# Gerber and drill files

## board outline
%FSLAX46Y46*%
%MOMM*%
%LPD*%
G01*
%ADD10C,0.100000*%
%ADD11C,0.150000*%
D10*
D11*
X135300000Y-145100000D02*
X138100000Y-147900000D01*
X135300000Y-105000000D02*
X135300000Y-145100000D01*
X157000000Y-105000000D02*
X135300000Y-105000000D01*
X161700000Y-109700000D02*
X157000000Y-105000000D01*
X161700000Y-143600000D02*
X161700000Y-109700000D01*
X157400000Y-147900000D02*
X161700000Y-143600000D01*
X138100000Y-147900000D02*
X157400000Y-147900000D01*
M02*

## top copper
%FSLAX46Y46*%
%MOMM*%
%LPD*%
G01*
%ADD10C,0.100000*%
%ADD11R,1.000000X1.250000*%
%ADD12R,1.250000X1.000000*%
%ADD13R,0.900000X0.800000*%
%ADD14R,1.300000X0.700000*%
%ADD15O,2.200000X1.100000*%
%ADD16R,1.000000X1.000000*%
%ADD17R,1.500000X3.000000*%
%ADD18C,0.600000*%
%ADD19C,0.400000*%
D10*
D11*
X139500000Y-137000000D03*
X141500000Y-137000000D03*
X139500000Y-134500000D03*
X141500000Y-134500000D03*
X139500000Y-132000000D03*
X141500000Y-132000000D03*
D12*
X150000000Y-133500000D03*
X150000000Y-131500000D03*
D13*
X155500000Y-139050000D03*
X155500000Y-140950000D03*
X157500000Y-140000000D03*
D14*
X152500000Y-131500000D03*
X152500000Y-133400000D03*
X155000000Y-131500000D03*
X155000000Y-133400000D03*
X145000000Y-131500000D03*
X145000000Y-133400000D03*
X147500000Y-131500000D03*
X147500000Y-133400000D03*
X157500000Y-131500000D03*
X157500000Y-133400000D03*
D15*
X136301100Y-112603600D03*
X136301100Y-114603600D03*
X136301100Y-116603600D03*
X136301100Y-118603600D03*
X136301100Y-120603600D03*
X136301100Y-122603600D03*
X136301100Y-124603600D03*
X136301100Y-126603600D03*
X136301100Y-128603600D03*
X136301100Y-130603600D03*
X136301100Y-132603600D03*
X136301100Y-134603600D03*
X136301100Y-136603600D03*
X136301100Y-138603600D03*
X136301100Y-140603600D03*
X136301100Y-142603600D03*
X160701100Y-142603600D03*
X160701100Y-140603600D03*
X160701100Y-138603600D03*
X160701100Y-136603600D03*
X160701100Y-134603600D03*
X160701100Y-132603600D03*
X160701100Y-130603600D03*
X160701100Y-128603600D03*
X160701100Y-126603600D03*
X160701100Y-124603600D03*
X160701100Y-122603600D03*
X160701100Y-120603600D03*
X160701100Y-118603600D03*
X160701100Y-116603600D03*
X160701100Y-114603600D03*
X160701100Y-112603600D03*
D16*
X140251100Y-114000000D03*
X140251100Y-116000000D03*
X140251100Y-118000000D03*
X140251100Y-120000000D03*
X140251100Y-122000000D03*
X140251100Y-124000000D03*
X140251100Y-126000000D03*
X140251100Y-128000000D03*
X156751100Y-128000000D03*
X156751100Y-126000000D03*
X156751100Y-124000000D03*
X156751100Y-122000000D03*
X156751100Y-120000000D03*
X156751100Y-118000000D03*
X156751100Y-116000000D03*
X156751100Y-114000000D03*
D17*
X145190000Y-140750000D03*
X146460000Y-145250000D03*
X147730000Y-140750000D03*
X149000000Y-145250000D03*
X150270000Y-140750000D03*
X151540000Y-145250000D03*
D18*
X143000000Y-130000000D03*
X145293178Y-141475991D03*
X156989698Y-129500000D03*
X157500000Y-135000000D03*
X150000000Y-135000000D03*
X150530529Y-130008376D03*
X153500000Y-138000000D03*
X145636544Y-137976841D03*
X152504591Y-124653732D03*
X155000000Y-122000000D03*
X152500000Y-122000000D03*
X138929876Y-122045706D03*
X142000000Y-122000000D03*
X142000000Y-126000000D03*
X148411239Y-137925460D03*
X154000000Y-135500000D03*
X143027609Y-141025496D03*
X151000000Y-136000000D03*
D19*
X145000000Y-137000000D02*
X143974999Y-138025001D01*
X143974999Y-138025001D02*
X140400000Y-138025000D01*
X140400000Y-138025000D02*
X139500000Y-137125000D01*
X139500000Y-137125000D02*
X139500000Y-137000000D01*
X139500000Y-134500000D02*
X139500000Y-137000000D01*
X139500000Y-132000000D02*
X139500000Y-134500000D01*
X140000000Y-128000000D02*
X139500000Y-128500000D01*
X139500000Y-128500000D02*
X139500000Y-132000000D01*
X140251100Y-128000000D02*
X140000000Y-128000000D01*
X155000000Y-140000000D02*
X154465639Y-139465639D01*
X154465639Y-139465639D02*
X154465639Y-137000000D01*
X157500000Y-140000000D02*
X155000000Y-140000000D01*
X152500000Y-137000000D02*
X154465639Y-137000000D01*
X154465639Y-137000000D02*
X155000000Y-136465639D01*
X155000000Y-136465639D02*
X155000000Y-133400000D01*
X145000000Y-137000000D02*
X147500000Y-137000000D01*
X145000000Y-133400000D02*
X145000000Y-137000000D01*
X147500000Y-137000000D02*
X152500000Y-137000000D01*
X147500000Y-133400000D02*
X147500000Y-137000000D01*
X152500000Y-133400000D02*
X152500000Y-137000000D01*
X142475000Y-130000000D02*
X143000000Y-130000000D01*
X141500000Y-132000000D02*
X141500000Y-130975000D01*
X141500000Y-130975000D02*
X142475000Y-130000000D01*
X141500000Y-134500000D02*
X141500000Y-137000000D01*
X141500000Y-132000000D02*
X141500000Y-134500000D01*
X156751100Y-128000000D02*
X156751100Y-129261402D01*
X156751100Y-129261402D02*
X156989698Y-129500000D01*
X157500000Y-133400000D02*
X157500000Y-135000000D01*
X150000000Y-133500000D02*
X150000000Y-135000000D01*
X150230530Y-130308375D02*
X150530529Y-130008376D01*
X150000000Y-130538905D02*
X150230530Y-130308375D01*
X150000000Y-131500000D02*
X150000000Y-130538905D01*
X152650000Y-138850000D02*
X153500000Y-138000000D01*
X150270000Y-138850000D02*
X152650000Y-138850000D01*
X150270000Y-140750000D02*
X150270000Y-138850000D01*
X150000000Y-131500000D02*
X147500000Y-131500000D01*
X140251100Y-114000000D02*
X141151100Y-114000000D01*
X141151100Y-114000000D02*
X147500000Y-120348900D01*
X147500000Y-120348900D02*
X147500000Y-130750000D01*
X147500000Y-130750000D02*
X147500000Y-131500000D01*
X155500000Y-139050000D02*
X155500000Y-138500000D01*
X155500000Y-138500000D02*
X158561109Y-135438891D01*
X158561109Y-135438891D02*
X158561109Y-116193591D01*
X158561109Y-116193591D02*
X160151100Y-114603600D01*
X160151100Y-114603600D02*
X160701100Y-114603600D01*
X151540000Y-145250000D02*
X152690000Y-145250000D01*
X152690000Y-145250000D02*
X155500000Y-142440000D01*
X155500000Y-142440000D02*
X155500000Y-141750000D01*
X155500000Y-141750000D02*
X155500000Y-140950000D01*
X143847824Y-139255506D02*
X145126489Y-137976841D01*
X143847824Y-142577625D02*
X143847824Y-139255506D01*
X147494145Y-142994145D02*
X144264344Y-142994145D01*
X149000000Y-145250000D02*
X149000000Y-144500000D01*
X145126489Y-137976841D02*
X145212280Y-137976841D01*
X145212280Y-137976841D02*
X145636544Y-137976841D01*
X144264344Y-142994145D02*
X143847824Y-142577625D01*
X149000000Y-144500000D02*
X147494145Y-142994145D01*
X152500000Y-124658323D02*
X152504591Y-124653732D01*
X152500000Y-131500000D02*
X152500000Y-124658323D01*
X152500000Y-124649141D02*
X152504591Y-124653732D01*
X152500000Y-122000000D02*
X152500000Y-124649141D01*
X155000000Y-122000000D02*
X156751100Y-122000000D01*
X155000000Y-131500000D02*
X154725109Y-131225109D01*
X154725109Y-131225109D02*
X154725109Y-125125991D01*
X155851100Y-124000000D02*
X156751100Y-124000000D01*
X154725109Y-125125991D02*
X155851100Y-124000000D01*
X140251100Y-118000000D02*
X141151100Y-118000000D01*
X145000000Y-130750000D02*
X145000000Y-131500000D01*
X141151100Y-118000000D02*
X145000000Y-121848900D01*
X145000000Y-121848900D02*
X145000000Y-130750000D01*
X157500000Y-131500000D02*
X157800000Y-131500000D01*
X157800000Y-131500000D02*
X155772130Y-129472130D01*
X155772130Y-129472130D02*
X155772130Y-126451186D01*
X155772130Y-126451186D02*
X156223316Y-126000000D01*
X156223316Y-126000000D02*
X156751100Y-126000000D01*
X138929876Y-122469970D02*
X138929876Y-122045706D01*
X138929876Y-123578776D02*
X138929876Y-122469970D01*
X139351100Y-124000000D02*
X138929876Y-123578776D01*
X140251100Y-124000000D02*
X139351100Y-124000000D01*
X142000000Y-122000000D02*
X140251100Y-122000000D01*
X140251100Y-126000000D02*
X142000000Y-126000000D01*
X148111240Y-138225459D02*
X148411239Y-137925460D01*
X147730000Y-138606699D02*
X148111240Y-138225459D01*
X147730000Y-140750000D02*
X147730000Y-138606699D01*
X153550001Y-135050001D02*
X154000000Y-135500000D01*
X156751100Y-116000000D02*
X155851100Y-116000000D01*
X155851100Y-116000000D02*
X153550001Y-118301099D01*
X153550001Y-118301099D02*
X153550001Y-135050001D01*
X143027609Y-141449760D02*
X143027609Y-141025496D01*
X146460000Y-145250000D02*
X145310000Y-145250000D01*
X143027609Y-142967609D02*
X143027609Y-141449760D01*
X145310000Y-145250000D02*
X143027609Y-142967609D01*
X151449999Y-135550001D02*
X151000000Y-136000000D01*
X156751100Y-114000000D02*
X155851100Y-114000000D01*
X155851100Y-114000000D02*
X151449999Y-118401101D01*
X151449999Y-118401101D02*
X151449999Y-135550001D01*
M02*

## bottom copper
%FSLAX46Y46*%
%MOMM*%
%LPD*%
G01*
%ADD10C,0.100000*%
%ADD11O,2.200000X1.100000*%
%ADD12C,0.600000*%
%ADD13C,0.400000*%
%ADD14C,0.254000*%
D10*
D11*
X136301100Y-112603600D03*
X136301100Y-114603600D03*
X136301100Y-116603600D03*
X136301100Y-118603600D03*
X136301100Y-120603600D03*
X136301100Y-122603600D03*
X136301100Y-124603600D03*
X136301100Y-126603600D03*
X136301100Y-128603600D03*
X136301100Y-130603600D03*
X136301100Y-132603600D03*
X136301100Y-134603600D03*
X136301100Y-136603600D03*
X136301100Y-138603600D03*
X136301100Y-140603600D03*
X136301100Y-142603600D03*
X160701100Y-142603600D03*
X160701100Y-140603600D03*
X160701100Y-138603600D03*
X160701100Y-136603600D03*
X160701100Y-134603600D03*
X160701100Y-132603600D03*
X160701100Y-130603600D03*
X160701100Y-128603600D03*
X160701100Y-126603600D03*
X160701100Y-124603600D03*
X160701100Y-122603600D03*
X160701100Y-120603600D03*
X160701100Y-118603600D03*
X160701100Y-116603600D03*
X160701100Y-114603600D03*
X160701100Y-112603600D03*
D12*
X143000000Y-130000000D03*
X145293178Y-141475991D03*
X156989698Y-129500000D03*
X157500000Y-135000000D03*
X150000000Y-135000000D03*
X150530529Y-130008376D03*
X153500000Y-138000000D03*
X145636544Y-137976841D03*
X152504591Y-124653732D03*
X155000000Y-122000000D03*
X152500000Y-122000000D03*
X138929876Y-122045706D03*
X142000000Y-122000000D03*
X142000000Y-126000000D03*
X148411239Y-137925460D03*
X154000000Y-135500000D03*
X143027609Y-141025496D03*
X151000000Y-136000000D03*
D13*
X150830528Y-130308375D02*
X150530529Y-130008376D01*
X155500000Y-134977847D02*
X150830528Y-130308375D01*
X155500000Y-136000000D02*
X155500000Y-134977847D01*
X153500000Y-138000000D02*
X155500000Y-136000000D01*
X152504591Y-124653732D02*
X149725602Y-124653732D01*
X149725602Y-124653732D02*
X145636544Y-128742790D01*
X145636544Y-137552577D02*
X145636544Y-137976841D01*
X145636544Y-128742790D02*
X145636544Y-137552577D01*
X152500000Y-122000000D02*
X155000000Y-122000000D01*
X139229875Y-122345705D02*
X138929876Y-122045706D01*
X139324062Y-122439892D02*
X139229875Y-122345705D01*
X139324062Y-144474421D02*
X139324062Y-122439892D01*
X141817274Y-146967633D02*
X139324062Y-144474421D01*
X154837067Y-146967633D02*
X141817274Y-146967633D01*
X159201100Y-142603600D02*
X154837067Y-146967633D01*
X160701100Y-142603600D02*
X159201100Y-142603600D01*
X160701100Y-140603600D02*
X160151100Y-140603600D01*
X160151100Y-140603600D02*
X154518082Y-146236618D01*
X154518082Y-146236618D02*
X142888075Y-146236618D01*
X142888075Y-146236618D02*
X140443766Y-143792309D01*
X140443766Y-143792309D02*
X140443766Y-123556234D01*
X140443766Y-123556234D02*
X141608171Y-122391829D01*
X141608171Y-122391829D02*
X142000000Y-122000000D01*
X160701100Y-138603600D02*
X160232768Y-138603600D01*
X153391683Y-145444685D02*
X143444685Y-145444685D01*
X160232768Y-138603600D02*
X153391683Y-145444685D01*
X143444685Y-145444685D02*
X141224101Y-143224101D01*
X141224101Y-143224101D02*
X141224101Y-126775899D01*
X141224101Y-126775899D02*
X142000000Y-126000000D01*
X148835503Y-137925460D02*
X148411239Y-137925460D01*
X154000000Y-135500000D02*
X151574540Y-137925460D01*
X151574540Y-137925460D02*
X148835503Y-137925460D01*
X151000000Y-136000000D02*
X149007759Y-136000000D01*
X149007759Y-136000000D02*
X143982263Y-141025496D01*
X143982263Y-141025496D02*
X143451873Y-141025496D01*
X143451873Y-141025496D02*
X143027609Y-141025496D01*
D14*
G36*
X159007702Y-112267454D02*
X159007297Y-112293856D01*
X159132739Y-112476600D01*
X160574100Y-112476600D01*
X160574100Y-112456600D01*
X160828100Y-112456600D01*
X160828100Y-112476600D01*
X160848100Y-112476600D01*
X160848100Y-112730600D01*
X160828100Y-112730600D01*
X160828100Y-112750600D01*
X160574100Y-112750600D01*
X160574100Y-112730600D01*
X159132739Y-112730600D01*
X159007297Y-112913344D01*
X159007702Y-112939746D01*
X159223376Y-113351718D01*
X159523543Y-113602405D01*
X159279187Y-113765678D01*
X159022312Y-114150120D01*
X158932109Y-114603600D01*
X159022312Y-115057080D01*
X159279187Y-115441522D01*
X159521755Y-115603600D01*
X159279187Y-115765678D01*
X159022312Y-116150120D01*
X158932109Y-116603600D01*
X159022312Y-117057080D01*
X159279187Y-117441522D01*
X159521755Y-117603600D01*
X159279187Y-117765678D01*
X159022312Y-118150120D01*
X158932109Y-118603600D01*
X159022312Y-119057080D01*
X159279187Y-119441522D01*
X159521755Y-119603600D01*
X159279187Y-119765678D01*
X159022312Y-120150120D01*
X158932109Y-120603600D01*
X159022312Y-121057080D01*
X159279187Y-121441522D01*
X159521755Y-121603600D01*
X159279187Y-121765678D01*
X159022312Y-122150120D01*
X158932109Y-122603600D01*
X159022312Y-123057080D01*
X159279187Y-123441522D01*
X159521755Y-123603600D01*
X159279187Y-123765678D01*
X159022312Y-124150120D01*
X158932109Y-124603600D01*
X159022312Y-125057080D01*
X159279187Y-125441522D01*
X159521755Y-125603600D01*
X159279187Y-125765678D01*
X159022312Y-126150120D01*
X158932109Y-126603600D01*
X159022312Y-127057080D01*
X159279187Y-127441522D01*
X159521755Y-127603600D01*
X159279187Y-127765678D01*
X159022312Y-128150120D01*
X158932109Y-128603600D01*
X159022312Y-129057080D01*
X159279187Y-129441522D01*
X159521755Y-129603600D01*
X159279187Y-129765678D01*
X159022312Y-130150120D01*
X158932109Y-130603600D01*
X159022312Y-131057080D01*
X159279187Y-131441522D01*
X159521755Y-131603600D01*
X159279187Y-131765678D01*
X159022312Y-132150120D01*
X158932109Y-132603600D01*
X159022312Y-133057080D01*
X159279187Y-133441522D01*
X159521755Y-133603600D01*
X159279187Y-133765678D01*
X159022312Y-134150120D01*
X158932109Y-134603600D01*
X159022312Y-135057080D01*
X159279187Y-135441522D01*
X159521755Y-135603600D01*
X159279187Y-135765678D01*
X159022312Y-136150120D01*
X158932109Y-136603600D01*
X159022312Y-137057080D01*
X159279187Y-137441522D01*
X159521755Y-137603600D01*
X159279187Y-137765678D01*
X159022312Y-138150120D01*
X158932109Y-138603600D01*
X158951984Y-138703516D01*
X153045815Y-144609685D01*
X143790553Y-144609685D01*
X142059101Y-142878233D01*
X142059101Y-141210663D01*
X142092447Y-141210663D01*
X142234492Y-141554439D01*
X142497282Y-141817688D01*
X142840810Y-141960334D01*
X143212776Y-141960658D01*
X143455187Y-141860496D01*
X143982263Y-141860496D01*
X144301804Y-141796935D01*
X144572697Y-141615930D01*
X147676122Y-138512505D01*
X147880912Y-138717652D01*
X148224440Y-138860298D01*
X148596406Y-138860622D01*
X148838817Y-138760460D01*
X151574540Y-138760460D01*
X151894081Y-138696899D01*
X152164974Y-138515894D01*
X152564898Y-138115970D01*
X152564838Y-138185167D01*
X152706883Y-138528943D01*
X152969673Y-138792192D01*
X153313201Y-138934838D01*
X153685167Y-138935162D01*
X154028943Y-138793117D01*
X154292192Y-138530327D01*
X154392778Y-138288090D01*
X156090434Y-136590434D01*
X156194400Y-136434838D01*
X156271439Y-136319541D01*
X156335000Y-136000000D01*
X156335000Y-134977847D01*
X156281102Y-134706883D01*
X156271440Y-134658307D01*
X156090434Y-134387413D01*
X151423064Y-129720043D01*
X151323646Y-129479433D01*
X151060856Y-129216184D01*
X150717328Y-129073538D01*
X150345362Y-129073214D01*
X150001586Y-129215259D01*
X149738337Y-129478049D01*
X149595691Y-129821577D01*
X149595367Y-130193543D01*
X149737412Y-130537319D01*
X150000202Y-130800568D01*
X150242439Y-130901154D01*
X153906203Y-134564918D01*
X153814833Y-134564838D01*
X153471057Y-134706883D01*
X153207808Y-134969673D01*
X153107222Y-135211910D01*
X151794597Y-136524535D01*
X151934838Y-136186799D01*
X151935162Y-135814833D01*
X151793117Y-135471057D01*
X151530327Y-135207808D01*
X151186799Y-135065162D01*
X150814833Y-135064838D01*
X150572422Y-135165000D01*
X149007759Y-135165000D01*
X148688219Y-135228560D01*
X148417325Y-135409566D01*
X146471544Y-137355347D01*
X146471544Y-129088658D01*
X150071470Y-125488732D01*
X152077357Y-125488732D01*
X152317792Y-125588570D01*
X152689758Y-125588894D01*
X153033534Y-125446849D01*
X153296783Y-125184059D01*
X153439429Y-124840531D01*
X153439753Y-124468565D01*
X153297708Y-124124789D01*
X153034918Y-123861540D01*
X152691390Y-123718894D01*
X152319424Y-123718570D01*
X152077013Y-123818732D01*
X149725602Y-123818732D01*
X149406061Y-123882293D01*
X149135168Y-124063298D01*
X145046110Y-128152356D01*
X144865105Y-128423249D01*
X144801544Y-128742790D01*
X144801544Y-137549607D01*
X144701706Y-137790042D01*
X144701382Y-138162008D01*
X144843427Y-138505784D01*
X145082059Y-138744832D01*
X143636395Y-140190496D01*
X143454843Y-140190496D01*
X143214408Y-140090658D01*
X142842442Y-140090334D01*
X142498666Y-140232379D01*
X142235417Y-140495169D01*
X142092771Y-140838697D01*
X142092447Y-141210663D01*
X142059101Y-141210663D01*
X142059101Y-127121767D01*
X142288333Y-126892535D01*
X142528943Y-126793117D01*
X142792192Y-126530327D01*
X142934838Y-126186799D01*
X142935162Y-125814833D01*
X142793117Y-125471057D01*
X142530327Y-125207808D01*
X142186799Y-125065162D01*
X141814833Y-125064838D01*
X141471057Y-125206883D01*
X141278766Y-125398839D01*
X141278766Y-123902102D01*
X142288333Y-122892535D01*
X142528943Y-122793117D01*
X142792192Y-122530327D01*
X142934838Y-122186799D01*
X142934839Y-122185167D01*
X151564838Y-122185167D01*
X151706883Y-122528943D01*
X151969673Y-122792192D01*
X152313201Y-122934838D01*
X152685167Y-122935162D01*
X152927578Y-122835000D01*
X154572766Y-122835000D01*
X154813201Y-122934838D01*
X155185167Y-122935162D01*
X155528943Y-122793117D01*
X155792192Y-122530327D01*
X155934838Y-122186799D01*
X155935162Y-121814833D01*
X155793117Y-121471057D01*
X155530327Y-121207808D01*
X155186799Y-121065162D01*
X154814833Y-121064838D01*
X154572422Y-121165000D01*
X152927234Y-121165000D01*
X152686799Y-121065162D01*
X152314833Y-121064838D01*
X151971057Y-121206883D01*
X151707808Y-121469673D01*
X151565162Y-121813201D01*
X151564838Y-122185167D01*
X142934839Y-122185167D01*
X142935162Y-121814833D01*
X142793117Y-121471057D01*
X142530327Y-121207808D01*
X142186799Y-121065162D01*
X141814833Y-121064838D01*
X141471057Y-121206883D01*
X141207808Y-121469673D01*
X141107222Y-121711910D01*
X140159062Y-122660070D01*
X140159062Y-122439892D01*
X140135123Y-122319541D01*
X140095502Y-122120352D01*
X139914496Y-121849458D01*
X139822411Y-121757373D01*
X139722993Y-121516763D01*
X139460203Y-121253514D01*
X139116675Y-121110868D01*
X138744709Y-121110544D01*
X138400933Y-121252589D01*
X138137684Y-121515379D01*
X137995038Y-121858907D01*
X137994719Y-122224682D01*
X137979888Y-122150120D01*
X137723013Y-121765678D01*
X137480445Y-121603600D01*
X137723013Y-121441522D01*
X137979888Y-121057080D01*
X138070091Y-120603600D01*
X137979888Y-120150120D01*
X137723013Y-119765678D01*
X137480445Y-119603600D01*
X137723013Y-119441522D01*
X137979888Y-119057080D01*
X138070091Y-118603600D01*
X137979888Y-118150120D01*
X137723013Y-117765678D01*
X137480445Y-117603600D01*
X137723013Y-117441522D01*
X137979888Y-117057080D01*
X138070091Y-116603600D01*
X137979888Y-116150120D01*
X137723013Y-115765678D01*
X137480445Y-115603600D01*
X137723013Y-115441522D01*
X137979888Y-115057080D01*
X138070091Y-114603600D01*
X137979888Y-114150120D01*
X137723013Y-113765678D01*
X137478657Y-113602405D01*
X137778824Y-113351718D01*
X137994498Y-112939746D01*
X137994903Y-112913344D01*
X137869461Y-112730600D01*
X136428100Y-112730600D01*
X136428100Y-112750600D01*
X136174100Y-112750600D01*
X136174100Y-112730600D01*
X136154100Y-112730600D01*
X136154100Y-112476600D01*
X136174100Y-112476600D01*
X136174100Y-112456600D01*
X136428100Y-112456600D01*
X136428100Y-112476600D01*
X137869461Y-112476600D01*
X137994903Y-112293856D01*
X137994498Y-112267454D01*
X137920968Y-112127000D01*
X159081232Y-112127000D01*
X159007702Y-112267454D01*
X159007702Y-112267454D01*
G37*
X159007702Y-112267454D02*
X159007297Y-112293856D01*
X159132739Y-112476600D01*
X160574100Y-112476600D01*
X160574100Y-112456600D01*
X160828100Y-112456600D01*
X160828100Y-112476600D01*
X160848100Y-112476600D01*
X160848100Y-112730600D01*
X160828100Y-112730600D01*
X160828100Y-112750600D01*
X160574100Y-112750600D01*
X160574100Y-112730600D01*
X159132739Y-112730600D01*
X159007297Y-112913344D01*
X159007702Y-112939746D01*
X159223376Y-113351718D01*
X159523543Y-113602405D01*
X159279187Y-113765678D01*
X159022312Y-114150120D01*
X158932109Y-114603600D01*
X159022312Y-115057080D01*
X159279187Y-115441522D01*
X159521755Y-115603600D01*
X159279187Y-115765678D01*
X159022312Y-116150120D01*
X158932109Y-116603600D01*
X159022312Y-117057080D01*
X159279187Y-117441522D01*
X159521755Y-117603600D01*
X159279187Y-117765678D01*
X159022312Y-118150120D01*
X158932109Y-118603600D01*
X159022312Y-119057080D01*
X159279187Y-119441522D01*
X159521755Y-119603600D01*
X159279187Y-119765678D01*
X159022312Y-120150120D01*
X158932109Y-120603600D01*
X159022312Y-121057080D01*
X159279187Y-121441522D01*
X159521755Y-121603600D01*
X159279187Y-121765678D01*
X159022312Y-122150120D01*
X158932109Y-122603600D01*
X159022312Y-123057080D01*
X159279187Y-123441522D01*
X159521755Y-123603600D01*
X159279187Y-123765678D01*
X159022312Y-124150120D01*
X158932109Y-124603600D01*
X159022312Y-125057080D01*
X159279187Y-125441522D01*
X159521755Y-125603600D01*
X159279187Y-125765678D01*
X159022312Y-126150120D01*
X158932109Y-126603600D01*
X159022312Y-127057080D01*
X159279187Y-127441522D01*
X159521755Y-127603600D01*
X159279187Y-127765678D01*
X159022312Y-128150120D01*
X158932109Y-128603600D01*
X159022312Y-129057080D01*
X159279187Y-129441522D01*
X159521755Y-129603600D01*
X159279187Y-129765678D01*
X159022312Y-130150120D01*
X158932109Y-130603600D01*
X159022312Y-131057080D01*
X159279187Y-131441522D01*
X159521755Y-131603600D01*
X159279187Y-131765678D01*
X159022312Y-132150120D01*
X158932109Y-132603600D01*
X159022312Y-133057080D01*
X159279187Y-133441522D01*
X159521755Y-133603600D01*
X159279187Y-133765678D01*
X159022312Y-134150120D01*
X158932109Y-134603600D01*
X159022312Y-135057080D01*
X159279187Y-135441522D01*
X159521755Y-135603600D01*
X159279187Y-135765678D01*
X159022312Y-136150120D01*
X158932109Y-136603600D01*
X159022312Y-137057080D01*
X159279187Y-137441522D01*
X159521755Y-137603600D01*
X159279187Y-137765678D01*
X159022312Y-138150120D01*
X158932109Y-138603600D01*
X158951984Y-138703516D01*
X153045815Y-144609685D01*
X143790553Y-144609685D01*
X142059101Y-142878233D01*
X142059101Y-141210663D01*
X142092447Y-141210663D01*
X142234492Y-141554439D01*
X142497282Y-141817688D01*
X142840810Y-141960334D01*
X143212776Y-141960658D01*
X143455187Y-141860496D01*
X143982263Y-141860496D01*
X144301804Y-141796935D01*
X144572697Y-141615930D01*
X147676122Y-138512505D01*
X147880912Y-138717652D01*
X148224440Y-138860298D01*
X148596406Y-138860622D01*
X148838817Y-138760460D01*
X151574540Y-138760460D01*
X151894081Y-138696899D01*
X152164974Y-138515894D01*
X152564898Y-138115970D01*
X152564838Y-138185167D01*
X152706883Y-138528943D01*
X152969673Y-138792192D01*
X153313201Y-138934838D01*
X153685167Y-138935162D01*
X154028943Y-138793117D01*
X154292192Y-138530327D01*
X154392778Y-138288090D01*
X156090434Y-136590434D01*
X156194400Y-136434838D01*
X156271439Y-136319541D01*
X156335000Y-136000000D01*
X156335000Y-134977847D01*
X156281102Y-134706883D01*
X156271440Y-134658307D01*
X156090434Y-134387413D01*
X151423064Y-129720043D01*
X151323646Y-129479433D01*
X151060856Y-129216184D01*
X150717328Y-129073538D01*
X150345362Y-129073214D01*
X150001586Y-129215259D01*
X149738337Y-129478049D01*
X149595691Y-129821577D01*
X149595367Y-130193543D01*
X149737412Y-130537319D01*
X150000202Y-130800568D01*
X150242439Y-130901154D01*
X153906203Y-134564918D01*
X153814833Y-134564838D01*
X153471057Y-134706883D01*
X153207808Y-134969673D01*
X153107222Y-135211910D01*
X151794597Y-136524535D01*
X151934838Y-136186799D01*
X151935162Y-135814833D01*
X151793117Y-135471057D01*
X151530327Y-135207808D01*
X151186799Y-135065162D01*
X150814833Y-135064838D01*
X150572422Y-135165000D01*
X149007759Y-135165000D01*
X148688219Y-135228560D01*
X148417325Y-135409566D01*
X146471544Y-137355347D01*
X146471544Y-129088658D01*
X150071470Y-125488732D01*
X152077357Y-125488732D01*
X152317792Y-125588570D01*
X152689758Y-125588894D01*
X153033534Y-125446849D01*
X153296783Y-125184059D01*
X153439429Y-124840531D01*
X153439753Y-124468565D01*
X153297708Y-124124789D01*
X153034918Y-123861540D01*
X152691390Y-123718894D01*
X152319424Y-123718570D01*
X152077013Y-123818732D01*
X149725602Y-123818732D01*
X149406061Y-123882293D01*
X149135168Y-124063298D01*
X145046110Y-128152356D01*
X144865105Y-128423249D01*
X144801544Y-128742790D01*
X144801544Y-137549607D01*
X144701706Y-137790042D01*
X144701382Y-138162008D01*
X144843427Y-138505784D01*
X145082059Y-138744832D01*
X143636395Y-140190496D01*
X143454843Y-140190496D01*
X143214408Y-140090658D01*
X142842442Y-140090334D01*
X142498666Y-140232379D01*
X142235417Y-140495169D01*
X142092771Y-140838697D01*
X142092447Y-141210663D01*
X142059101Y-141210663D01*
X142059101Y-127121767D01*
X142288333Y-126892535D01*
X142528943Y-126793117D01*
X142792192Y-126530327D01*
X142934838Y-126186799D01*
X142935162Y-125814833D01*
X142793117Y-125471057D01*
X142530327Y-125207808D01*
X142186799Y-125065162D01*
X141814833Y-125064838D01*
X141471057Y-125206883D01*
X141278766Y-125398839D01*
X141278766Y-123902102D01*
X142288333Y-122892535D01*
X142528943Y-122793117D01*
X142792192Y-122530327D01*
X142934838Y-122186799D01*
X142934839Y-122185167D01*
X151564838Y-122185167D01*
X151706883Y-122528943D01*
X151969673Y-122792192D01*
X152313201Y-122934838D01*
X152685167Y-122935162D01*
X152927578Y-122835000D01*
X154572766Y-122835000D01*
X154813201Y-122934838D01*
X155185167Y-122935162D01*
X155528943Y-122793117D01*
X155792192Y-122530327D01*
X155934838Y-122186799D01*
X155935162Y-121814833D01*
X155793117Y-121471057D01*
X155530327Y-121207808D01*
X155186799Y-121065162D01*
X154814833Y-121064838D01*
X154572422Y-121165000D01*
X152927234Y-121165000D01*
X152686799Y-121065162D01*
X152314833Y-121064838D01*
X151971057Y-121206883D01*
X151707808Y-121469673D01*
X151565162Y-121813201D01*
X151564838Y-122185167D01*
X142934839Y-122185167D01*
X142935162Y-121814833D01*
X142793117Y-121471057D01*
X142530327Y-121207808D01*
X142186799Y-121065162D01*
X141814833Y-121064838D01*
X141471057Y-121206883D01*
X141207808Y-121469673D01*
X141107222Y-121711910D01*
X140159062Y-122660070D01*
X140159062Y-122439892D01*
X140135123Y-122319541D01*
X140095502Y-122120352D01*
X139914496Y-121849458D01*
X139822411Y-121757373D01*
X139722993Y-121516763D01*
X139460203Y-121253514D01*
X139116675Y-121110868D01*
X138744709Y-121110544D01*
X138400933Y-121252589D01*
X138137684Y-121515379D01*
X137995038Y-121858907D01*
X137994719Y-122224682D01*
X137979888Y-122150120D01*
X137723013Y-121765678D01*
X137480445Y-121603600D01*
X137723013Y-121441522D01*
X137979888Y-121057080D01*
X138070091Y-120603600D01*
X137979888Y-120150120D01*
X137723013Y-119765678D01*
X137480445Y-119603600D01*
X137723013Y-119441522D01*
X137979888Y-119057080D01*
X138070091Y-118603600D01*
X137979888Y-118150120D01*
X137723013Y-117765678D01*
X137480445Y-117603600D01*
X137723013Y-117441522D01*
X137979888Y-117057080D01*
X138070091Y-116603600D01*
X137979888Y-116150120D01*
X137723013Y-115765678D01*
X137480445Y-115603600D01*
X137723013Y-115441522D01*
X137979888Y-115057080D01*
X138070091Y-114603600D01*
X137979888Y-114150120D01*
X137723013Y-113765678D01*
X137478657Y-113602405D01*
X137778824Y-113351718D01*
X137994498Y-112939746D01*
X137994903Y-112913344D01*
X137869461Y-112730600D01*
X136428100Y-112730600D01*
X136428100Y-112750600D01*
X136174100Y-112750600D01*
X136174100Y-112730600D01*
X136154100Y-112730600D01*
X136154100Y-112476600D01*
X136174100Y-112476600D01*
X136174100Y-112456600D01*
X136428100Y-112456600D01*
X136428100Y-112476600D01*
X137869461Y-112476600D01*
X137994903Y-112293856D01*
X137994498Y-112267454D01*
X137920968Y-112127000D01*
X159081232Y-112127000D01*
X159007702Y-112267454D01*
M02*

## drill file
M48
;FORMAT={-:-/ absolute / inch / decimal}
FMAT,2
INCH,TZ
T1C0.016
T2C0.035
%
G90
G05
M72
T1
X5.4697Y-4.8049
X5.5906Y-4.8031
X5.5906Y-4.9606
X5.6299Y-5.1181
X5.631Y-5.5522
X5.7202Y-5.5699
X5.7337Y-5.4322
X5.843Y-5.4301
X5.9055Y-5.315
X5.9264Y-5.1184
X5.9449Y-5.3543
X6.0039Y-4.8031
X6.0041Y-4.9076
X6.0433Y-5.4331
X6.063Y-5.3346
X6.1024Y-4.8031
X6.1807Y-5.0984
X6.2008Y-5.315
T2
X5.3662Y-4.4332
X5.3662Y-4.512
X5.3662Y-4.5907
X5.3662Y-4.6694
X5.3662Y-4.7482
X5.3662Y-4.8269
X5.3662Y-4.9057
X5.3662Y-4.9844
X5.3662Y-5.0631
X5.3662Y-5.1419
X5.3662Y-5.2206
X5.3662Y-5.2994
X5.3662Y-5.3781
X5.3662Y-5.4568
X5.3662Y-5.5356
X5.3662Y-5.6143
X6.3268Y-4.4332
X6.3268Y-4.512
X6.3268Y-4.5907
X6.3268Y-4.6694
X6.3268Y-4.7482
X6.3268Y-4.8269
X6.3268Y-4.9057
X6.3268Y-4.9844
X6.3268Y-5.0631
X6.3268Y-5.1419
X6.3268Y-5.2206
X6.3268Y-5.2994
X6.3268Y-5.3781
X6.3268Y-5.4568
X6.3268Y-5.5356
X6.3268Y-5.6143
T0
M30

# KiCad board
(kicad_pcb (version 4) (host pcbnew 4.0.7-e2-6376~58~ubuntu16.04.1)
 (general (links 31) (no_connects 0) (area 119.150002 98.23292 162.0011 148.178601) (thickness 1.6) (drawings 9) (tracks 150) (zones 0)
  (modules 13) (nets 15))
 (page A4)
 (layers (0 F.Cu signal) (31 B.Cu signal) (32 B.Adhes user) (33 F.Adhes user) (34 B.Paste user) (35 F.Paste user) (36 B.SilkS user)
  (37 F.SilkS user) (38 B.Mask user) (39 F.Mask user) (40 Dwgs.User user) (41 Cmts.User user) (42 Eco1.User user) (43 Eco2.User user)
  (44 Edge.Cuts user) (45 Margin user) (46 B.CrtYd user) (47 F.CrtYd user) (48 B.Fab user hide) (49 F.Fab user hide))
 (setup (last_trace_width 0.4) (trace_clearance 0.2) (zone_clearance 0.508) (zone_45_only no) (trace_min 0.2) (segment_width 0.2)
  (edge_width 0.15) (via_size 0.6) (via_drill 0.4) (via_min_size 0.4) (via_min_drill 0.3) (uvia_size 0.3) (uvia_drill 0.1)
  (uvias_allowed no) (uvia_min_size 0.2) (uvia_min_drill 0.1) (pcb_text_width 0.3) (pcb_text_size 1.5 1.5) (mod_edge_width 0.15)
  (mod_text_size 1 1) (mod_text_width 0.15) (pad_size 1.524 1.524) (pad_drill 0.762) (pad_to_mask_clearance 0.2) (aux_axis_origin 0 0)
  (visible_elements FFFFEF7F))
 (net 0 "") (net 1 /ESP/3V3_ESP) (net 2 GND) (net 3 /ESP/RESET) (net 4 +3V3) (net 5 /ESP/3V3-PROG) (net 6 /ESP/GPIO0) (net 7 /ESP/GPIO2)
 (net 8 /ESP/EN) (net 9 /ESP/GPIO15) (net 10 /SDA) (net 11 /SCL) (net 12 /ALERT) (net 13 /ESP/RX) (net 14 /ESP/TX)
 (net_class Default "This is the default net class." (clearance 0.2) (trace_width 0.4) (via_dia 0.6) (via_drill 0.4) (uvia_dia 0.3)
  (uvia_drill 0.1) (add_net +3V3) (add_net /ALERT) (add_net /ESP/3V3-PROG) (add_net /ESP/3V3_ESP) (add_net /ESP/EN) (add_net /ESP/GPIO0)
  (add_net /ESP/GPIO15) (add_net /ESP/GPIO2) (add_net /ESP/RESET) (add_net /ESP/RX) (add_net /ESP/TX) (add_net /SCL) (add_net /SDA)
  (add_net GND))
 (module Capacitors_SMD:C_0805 (layer F.Cu) (at 140.5 137)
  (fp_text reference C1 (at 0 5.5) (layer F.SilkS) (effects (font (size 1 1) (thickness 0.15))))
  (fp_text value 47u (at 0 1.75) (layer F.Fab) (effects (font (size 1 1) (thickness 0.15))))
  (pad 1 smd rect (at -1 0) (size 1 1.25) (layers F.Cu F.Paste F.Mask) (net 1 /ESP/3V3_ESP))
  (pad 2 smd rect (at 1 0) (size 1 1.25) (layers F.Cu F.Paste F.Mask) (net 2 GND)))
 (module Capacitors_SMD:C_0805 (layer F.Cu) (at 140.5 134.5)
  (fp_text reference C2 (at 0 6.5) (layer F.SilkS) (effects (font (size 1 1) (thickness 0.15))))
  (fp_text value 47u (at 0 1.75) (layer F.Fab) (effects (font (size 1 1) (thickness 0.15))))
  (pad 1 smd rect (at -1 0) (size 1 1.25) (layers F.Cu F.Paste F.Mask) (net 1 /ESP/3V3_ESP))
  (pad 2 smd rect (at 1 0) (size 1 1.25) (layers F.Cu F.Paste F.Mask) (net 2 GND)))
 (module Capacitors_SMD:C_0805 (layer F.Cu) (at 140.5 132)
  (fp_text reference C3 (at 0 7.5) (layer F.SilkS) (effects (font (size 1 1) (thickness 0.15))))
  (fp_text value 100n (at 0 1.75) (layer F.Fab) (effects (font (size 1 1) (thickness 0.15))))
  (pad 1 smd rect (at -1 0) (size 1 1.25) (layers F.Cu F.Paste F.Mask) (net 1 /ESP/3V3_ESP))
  (pad 2 smd rect (at 1 0) (size 1 1.25) (layers F.Cu F.Paste F.Mask) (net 2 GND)))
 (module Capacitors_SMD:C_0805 (layer F.Cu) (at 150 132.5 90)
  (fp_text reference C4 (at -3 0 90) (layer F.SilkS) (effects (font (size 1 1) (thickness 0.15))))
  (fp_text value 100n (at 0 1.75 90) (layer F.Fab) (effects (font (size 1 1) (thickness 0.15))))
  (pad 1 smd rect (at -1 0 90) (size 1 1.25) (layers F.Cu F.Paste F.Mask) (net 2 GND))
  (pad 2 smd rect (at 1 0 90) (size 1 1.25) (layers F.Cu F.Paste F.Mask) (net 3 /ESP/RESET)))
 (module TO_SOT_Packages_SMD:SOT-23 (layer F.Cu) (at 156.5 140)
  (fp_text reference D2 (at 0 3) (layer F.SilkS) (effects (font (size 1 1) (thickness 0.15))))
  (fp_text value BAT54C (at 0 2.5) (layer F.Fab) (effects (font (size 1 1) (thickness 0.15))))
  (pad 1 smd rect (at -1 -0.95) (size 0.9 0.8) (layers F.Cu F.Paste F.Mask) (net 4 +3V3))
  (pad 2 smd rect (at -1 0.95) (size 0.9 0.8) (layers F.Cu F.Paste F.Mask) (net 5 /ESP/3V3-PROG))
  (pad 3 smd rect (at 1 0) (size 0.9 0.8) (layers F.Cu F.Paste F.Mask) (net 1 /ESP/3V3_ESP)))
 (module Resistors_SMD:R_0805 (layer F.Cu) (at 152.5 132.45 270)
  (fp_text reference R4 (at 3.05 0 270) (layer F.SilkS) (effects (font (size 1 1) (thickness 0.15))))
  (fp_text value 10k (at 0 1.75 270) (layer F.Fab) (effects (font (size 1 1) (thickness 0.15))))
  (pad 1 smd rect (at -0.95 0 270) (size 0.7 1.3) (layers F.Cu F.Paste F.Mask) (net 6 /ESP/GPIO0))
  (pad 2 smd rect (at 0.95 0 270) (size 0.7 1.3) (layers F.Cu F.Paste F.Mask) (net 1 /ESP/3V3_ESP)))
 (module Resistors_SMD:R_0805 (layer F.Cu) (at 155 132.45 270)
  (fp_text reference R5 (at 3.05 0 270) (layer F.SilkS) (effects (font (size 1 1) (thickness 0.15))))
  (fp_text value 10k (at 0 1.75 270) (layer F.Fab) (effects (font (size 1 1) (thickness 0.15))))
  (pad 1 smd rect (at -0.95 0 270) (size 0.7 1.3) (layers F.Cu F.Paste F.Mask) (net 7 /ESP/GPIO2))
  (pad 2 smd rect (at 0.95 0 270) (size 0.7 1.3) (layers F.Cu F.Paste F.Mask) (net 1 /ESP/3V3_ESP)))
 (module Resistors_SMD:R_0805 (layer F.Cu) (at 145 132.45 270)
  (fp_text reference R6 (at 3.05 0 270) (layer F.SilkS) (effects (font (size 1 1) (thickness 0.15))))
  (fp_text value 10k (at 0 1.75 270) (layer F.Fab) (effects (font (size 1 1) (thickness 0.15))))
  (pad 1 smd rect (at -0.95 0 270) (size 0.7 1.3) (layers F.Cu F.Paste F.Mask) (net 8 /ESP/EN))
  (pad 2 smd rect (at 0.95 0 270) (size 0.7 1.3) (layers F.Cu F.Paste F.Mask) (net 1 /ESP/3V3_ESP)))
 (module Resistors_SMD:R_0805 (layer F.Cu) (at 147.5 132.45 270)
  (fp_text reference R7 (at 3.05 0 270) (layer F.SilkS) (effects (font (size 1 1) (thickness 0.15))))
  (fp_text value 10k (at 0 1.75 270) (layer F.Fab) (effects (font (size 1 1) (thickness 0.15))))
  (pad 1 smd rect (at -0.95 0 270) (size 0.7 1.3) (layers F.Cu F.Paste F.Mask) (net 3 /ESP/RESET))
  (pad 2 smd rect (at 0.95 0 270) (size 0.7 1.3) (layers F.Cu F.Paste F.Mask) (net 1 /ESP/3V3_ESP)))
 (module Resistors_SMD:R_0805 (layer F.Cu) (at 157.5 132.45 270)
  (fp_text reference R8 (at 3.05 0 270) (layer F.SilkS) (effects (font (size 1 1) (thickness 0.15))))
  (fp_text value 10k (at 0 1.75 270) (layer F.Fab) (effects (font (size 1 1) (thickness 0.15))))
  (pad 1 smd rect (at -0.95 0 270) (size 0.7 1.3) (layers F.Cu F.Paste F.Mask) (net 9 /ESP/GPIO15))
  (pad 2 smd rect (at 0.95 0 270) (size 0.7 1.3) (layers F.Cu F.Paste F.Mask) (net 2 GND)))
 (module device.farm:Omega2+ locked (layer F.Cu) (at 148.5011 105.0036)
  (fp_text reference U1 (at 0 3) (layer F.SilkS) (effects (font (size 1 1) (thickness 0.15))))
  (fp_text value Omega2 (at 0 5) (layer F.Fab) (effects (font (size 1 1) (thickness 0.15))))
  (pad 1 thru_hole oval (at -12.2 7.6) (size 2.2 1.1) (drill 0.9) (layers *.Cu *.Mask) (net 2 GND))
  (pad 2 thru_hole oval (at -12.2 9.6) (size 2.2 1.1) (drill 0.9) (layers *.Cu *.Mask))
  (pad 3 thru_hole oval (at -12.2 11.6) (size 2.2 1.1) (drill 0.9) (layers *.Cu *.Mask))
  (pad 4 thru_hole oval (at -12.2 13.6) (size 2.2 1.1) (drill 0.9) (layers *.Cu *.Mask))
  (pad 5 thru_hole oval (at -12.2 15.6) (size 2.2 1.1) (drill 0.9) (layers *.Cu *.Mask))
  (pad 6 thru_hole oval (at -12.2 17.6) (size 2.2 1.1) (drill 0.9) (layers *.Cu *.Mask))
  (pad 7 thru_hole oval (at -12.2 19.6) (size 2.2 1.1) (drill 0.9) (layers *.Cu *.Mask))
  (pad 8 thru_hole oval (at -12.2 21.6) (size 2.2 1.1) (drill 0.9) (layers *.Cu *.Mask))
  (pad 9 thru_hole oval (at -12.2 23.6) (size 2.2 1.1) (drill 0.9) (layers *.Cu *.Mask))
  (pad 10 thru_hole oval (at -12.2 25.6) (size 2.2 1.1) (drill 0.9) (layers *.Cu *.Mask))
  (pad 11 thru_hole oval (at -12.2 27.6) (size 2.2 1.1) (drill 0.9) (layers *.Cu *.Mask))
  (pad 12 thru_hole oval (at -12.2 29.6) (size 2.2 1.1) (drill 0.9) (layers *.Cu *.Mask))
  (pad 13 thru_hole oval (at -12.2 31.6) (size 2.2 1.1) (drill 0.9) (layers *.Cu *.Mask))
  (pad 14 thru_hole oval (at -12.2 33.6) (size 2.2 1.1) (drill 0.9) (layers *.Cu *.Mask))
  (pad 15 thru_hole oval (at -12.2 35.6) (size 2.2 1.1) (drill 0.9) (layers *.Cu *.Mask))
  (pad 16 thru_hole oval (at -12.2 37.6) (size 2.2 1.1) (drill 0.9) (layers *.Cu *.Mask))
  (pad 17 thru_hole oval (at 12.2 37.6) (size 2.2 1.1) (drill 0.9) (layers *.Cu *.Mask) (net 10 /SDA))
  (pad 18 thru_hole oval (at 12.2 35.6) (size 2.2 1.1) (drill 0.9) (layers *.Cu *.Mask) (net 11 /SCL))
  (pad 19 thru_hole oval (at 12.2 33.6) (size 2.2 1.1) (drill 0.9) (layers *.Cu *.Mask) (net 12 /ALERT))
  (pad 20 thru_hole oval (at 12.2 31.6) (size 2.2 1.1) (drill 0.9) (layers *.Cu *.Mask))
  (pad 21 thru_hole oval (at 12.2 29.6) (size 2.2 1.1) (drill 0.9) (layers *.Cu *.Mask))
  (pad 22 thru_hole oval (at 12.2 27.6) (size 2.2 1.1) (drill 0.9) (layers *.Cu *.Mask))
  (pad 23 thru_hole oval (at 12.2 25.6) (size 2.2 1.1) (drill 0.9) (layers *.Cu *.Mask))
  (pad 24 thru_hole oval (at 12.2 23.6) (size 2.2 1.1) (drill 0.9) (layers *.Cu *.Mask))
  (pad 25 thru_hole oval (at 12.2 21.6) (size 2.2 1.1) (drill 0.9) (layers *.Cu *.Mask))
  (pad 26 thru_hole oval (at 12.2 19.6) (size 2.2 1.1) (drill 0.9) (layers *.Cu *.Mask))
  (pad 27 thru_hole oval (at 12.2 17.6) (size 2.2 1.1) (drill 0.9) (layers *.Cu *.Mask))
  (pad 28 thru_hole oval (at 12.2 15.6) (size 2.2 1.1) (drill 0.9) (layers *.Cu *.Mask))
  (pad 29 thru_hole oval (at 12.2 13.6) (size 2.2 1.1) (drill 0.9) (layers *.Cu *.Mask))
  (pad 30 thru_hole oval (at 12.2 11.6) (size 2.2 1.1) (drill 0.9) (layers *.Cu *.Mask))
  (pad 31 thru_hole oval (at 12.2 9.6) (size 2.2 1.1) (drill 0.9) (layers *.Cu *.Mask) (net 4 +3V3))
  (pad 32 thru_hole oval (at 12.2 7.6) (size 2.2 1.1) (drill 0.9) (layers *.Cu *.Mask) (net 2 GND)))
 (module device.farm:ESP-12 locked (layer F.Cu) (at 148.5011 129.5)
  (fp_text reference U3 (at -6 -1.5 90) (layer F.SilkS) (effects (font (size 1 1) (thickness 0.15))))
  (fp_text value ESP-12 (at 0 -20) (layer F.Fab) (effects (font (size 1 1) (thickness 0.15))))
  (pad 1 smd rect (at -8.25 -15.5) (size 1 1) (layers F.Cu F.Paste F.Mask) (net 3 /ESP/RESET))
  (pad 2 smd rect (at -8.25 -13.5) (size 1 1) (layers F.Cu F.Paste F.Mask))
  (pad 3 smd rect (at -8.25 -11.5) (size 1 1) (layers F.Cu F.Paste F.Mask) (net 8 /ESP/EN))
  (pad 4 smd rect (at -8.25 -9.5) (size 1 1) (layers F.Cu F.Paste F.Mask))
  (pad 5 smd rect (at -8.25 -7.5) (size 1 1) (layers F.Cu F.Paste F.Mask) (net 11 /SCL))
  (pad 6 smd rect (at -8.25 -5.5) (size 1 1) (layers F.Cu F.Paste F.Mask) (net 10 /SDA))
  (pad 7 smd rect (at -8.25 -3.5) (size 1 1) (layers F.Cu F.Paste F.Mask) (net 12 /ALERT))
  (pad 8 smd rect (at -8.25 -1.5) (size 1 1) (layers F.Cu F.Paste F.Mask) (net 1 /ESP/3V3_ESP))
  (pad 9 smd rect (at 8.25 -1.5) (size 1 1) (layers F.Cu F.Paste F.Mask) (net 2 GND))
  (pad 10 smd rect (at 8.25 -3.5) (size 1 1) (layers F.Cu F.Paste F.Mask) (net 9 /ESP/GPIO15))
  (pad 11 smd rect (at 8.25 -5.5) (size 1 1) (layers F.Cu F.Paste F.Mask) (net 7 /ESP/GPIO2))
  (pad 12 smd rect (at 8.25 -7.5) (size 1 1) (layers F.Cu F.Paste F.Mask) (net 6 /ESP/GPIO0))
  (pad 13 smd rect (at 8.25 -9.5) (size 1 1) (layers F.Cu F.Paste F.Mask))
  (pad 14 smd rect (at 8.25 -11.5) (size 1 1) (layers F.Cu F.Paste F.Mask))
  (pad 15 smd rect (at 8.25 -13.5) (size 1 1) (layers F.Cu F.Paste F.Mask) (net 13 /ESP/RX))
  (pad 16 smd rect (at 8.25 -15.5) (size 1 1) (layers F.Cu F.Paste F.Mask) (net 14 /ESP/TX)))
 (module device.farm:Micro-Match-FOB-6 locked (layer F.Cu) (at 148.365 143)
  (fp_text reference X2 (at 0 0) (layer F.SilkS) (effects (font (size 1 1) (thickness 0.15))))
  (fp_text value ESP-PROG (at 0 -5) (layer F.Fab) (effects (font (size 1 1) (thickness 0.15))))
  (pad 1 smd rect (at -3.175 -2.25) (size 1.5 3) (layers F.Cu F.Paste F.Mask) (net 2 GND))
  (pad 2 smd rect (at -1.905 2.25) (size 1.5 3) (layers F.Cu F.Paste F.Mask) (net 14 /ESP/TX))
  (pad 3 smd rect (at -0.635 -2.25) (size 1.5 3) (layers F.Cu F.Paste F.Mask) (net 13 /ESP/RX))
  (pad 4 smd rect (at 0.635 2.25) (size 1.5 3) (layers F.Cu F.Paste F.Mask) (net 6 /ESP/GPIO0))
  (pad 5 smd rect (at 1.905 -2.25) (size 1.5 3) (layers F.Cu F.Paste F.Mask) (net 3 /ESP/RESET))
  (pad 6 smd rect (at 3.175 2.25) (size 1.5 3) (layers F.Cu F.Paste F.Mask) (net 5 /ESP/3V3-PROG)))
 (gr_line (start 135.3 145.1) (end 138.1 147.9) (layer Edge.Cuts) (width 0.15))
 (gr_line (start 135.3 105) (end 135.3 145.1) (layer Edge.Cuts) (width 0.15))
 (gr_line (start 157 105) (end 135.3 105) (layer Edge.Cuts) (width 0.15))
 (gr_line (start 161.7 109.7) (end 157 105) (layer Edge.Cuts) (width 0.15))
 (gr_line (start 161.7 143.6) (end 161.7 109.7) (layer Edge.Cuts) (width 0.15))
 (gr_line (start 157.4 147.9) (end 161.7 143.6) (layer Edge.Cuts) (width 0.15))
 (gr_line (start 138.1 147.9) (end 157.4 147.9) (layer Edge.Cuts) (width 0.15))
 (segment (start 145 137) (end 143.974999 138.025001) (width 0.4) (layer F.Cu) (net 1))
 (segment (start 143.974999 138.025001) (end 140.4 138.025) (width 0.4) (layer F.Cu) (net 1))
 (segment (start 140.4 138.025) (end 139.5 137.125) (width 0.4) (layer F.Cu) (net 1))
 (segment (start 139.5 137.125) (end 139.5 137) (width 0.4) (layer F.Cu) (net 1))
 (segment (start 139.5 134.5) (end 139.5 137) (width 0.4) (layer F.Cu) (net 1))
 (segment (start 139.5 132) (end 139.5 134.5) (width 0.4) (layer F.Cu) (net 1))
 (segment (start 140 128) (end 139.5 128.5) (width 0.4) (layer F.Cu) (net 1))
 (segment (start 139.5 128.5) (end 139.5 132) (width 0.4) (layer F.Cu) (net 1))
 (segment (start 140.2511 128) (end 140 128) (width 0.4) (layer F.Cu) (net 1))
 (segment (start 155 140) (end 154.465639 139.465639) (width 0.4) (layer F.Cu) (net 1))
 (segment (start 154.465639 139.465639) (end 154.465639 137) (width 0.4) (layer F.Cu) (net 1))
 (segment (start 157.5 140) (end 155 140) (width 0.4) (layer F.Cu) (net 1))
 (segment (start 152.5 137) (end 154.465639 137) (width 0.4) (layer F.Cu) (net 1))
 (segment (start 154.465639 137) (end 155 136.465639) (width 0.4) (layer F.Cu) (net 1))
 (segment (start 155 136.465639) (end 155 133.4) (width 0.4) (layer F.Cu) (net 1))
 (segment (start 145 137) (end 147.5 137) (width 0.4) (layer F.Cu) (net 1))
 (segment (start 145 133.4) (end 145 137) (width 0.4) (layer F.Cu) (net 1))
 (segment (start 147.5 137) (end 152.5 137) (width 0.4) (layer F.Cu) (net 1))
 (segment (start 147.5 133.4) (end 147.5 137) (width 0.4) (layer F.Cu) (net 1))
 (segment (start 152.5 133.4) (end 152.5 137) (width 0.4) (layer F.Cu) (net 1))
 (segment (start 142.475 130) (end 143 130) (width 0.4) (layer F.Cu) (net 2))
 (via (at 143 130) (size 0.6) (drill 0.4) (layers F.Cu B.Cu) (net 2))
 (segment (start 141.5 132) (end 141.5 130.975) (width 0.4) (layer F.Cu) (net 2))
 (segment (start 141.5 130.975) (end 142.475 130) (width 0.4) (layer F.Cu) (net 2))
 (segment (start 141.5 134.5) (end 141.5 137) (width 0.4) (layer F.Cu) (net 2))
 (segment (start 141.5 132) (end 141.5 134.5) (width 0.4) (layer F.Cu) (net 2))
 (via (at 145.293178 141.475991) (size 0.6) (drill 0.4) (layers F.Cu B.Cu) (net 2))
 (segment (start 156.7511 128) (end 156.7511 129.261402) (width 0.4) (layer F.Cu) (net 2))
 (segment (start 156.7511 129.261402) (end 156.989698 129.5) (width 0.4) (layer F.Cu) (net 2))
 (via (at 156.989698 129.5) (size 0.6) (drill 0.4) (layers F.Cu B.Cu) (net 2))
 (via (at 157.5 135) (size 0.6) (drill 0.4) (layers F.Cu B.Cu) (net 2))
 (segment (start 157.5 133.4) (end 157.5 135) (width 0.4) (layer F.Cu) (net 2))
 (via (at 150 135) (size 0.6) (drill 0.4) (layers F.Cu B.Cu) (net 2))
 (segment (start 150 133.5) (end 150 135) (width 0.4) (layer F.Cu) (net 2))
 (segment (start 150.830528 130.308375) (end 150.530529 130.008376) (width 0.4) (layer B.Cu) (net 3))
 (segment (start 155.5 134.977847) (end 150.830528 130.308375) (width 0.4) (layer B.Cu) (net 3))
 (segment (start 155.5 136) (end 155.5 134.977847) (width 0.4) (layer B.Cu) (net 3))
 (segment (start 153.5 138) (end 155.5 136) (width 0.4) (layer B.Cu) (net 3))
 (segment (start 150.23053 130.308375) (end 150.530529 130.008376) (width 0.4) (layer F.Cu) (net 3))
 (segment (start 150 130.538905) (end 150.23053 130.308375) (width 0.4) (layer F.Cu) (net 3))
 (segment (start 150 131.5) (end 150 130.538905) (width 0.4) (layer F.Cu) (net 3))
 (via (at 150.530529 130.008376) (size 0.6) (drill 0.4) (layers F.Cu B.Cu) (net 3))
 (segment (start 152.65 138.85) (end 153.5 138) (width 0.4) (layer F.Cu) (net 3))
 (via (at 153.5 138) (size 0.6) (drill 0.4) (layers F.Cu B.Cu) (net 3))
 (segment (start 150.27 138.85) (end 152.65 138.85) (width 0.4) (layer F.Cu) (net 3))
 (segment (start 150.27 140.75) (end 150.27 138.85) (width 0.4) (layer F.Cu) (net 3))
 (segment (start 150 131.5) (end 147.5 131.5) (width 0.4) (layer F.Cu) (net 3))
 (segment (start 140.2511 114) (end 141.1511 114) (width 0.4) (layer F.Cu) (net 3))
 (segment (start 141.1511 114) (end 147.5 120.3489) (width 0.4) (layer F.Cu) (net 3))
 (segment (start 147.5 120.3489) (end 147.5 130.75) (width 0.4) (layer F.Cu) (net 3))
 (segment (start 147.5 130.75) (end 147.5 131.5) (width 0.4) (layer F.Cu) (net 3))
 (segment (start 155.5 139.05) (end 155.5 138.5) (width 0.4) (layer F.Cu) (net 4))
 (segment (start 155.5 138.5) (end 158.561109 135.438891) (width 0.4) (layer F.Cu) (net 4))
 (segment (start 158.561109 135.438891) (end 158.561109 116.193591) (width 0.4) (layer F.Cu) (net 4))
 (segment (start 158.561109 116.193591) (end 160.1511 114.6036) (width 0.4) (layer F.Cu) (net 4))
 (segment (start 160.1511 114.6036) (end 160.7011 114.6036) (width 0.4) (layer F.Cu) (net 4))
 (segment (start 151.54 145.25) (end 152.69 145.25) (width 0.4) (layer F.Cu) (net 5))
 (segment (start 152.69 145.25) (end 155.5 142.44) (width 0.4) (layer F.Cu) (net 5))
 (segment (start 155.5 142.44) (end 155.5 141.75) (width 0.4) (layer F.Cu) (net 5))
 (segment (start 155.5 141.75) (end 155.5 140.95) (width 0.4) (layer F.Cu) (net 5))
 (segment (start 152.504591 124.653732) (end 149.725602 124.653732) (width 0.4) (layer B.Cu) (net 6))
 (segment (start 149.725602 124.653732) (end 145.636544 128.74279) (width 0.4) (layer B.Cu) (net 6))
 (segment (start 145.636544 137.552577) (end 145.636544 137.976841) (width 0.4) (layer B.Cu) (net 6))
 (segment (start 145.636544 128.74279) (end 145.636544 137.552577) (width 0.4) (layer B.Cu) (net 6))
 (segment (start 143.847824 139.255506) (end 145.126489 137.976841) (width 0.4) (layer F.Cu) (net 6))
 (segment (start 143.847824 142.577625) (end 143.847824 139.255506) (width 0.4) (layer F.Cu) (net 6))
 (segment (start 147.494145 142.994145) (end 144.264344 142.994145) (width 0.4) (layer F.Cu) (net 6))
 (segment (start 149 145.25) (end 149 144.5) (width 0.4) (layer F.Cu) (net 6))
 (segment (start 145.126489 137.976841) (end 145.21228 137.976841) (width 0.4) (layer F.Cu) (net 6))
 (segment (start 145.21228 137.976841) (end 145.636544 137.976841) (width 0.4) (layer F.Cu) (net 6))
 (segment (start 144.264344 142.994145) (end 143.847824 142.577625) (width 0.4) (layer F.Cu) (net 6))
 (segment (start 149 144.5) (end 147.494145 142.994145) (width 0.4) (layer F.Cu) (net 6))
 (via (at 145.636544 137.976841) (size 0.6) (drill 0.4) (layers F.Cu B.Cu) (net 6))
 (segment (start 152.5 124.658323) (end 152.504591 124.653732) (width 0.4) (layer F.Cu) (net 6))
 (segment (start 152.5 131.5) (end 152.5 124.658323) (width 0.4) (layer F.Cu) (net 6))
 (segment (start 152.5 124.649141) (end 152.504591 124.653732) (width 0.4) (layer F.Cu) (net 6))
 (segment (start 152.5 122) (end 152.5 124.649141) (width 0.4) (layer F.Cu) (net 6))
 (via (at 152.504591 124.653732) (size 0.6) (drill 0.4) (layers F.Cu B.Cu) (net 6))
 (segment (start 155 122) (end 156.7511 122) (width 0.4) (layer F.Cu) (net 6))
 (via (at 155 122) (size 0.6) (drill 0.4) (layers F.Cu B.Cu) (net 6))
 (segment (start 152.5 122) (end 155 122) (width 0.4) (layer B.Cu) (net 6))
 (via (at 152.5 122) (size 0.6) (drill 0.4) (layers F.Cu B.Cu) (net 6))
 (segment (start 155 131.5) (end 154.725109 131.225109) (width 0.4) (layer F.Cu) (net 7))
 (segment (start 154.725109 131.225109) (end 154.725109 125.125991) (width 0.4) (layer F.Cu) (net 7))
 (segment (start 155.8511 124) (end 156.7511 124) (width 0.4) (layer F.Cu) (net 7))
 (segment (start 154.725109 125.125991) (end 155.8511 124) (width 0.4) (layer F.Cu) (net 7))
 (segment (start 140.2511 118) (end 141.1511 118) (width 0.4) (layer F.Cu) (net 8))
 (segment (start 145 130.75) (end 145 131.5) (width 0.4) (layer F.Cu) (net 8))
 (segment (start 141.1511 118) (end 145 121.8489) (width 0.4) (layer F.Cu) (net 8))
 (segment (start 145 121.8489) (end 145 130.75) (width 0.4) (layer F.Cu) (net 8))
 (segment (start 157.5 131.5) (end 157.8 131.5) (width 0.4) (layer F.Cu) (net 9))
 (segment (start 157.8 131.5) (end 155.77213 129.47213) (width 0.4) (layer F.Cu) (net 9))
 (segment (start 155.77213 129.47213) (end 155.77213 126.451186) (width 0.4) (layer F.Cu) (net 9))
 (segment (start 155.77213 126.451186) (end 156.223316 126) (width 0.4) (layer F.Cu) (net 9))
 (segment (start 156.223316 126) (end 156.7511 126) (width 0.4) (layer F.Cu) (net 9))
 (segment (start 139.229875 122.345705) (end 138.929876 122.045706) (width 0.4) (layer B.Cu) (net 10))
 (segment (start 139.324062 122.439892) (end 139.229875 122.345705) (width 0.4) (layer B.Cu) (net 10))
 (segment (start 139.324062 144.474421) (end 139.324062 122.439892) (width 0.4) (layer B.Cu) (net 10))
 (segment (start 141.817274 146.967633) (end 139.324062 144.474421) (width 0.4) (layer B.Cu) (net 10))
 (segment (start 154.837067 146.967633) (end 141.817274 146.967633) (width 0.4) (layer B.Cu) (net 10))
 (segment (start 159.2011 142.6036) (end 154.837067 146.967633) (width 0.4) (layer B.Cu) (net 10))
 (segment (start 138.929876 122.46997) (end 138.929876 122.045706) (width 0.4) (layer F.Cu) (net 10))
 (segment (start 138.929876 123.578776) (end 138.929876 122.46997) (width 0.4) (layer F.Cu) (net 10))
 (segment (start 139.3511 124) (end 138.929876 123.578776) (width 0.4) (layer F.Cu) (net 10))
 (segment (start 140.2511 124) (end 139.3511 124) (width 0.4) (layer F.Cu) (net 10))
 (segment (start 160.7011 142.6036) (end 159.2011 142.6036) (width 0.4) (layer B.Cu) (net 10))
 (via (at 138.929876 122.045706) (size 0.6) (drill 0.4) (layers F.Cu B.Cu) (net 10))
 (segment (start 160.7011 140.6036) (end 160.1511 140.6036) (width 0.4) (layer B.Cu) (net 11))
 (segment (start 160.1511 140.6036) (end 154.518082 146.236618) (width 0.4) (layer B.Cu) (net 11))
 (segment (start 154.518082 146.236618) (end 142.888075 146.236618) (width 0.4) (layer B.Cu) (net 11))
 (segment (start 142.888075 146.236618) (end 140.443766 143.792309) (width 0.4) (layer B.Cu) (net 11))
 (segment (start 140.443766 143.792309) (end 140.443766 123.556234) (width 0.4) (layer B.Cu) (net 11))
 (segment (start 140.443766 123.556234) (end 141.608171 122.391829) (width 0.4) (layer B.Cu) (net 11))
 (segment (start 141.608171 122.391829) (end 142 122) (width 0.4) (layer B.Cu) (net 11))
 (segment (start 142 122) (end 140.2511 122) (width 0.4) (layer F.Cu) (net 11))
 (via (at 142 122) (size 0.6) (drill 0.4) (layers F.Cu B.Cu) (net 11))
 (segment (start 160.7011 138.6036) (end 160.232768 138.6036) (width 0.4) (layer B.Cu) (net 12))
 (segment (start 153.391683 145.444685) (end 143.444685 145.444685) (width 0.4) (layer B.Cu) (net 12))
 (segment (start 160.232768 138.6036) (end 153.391683 145.444685) (width 0.4) (layer B.Cu) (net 12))
 (segment (start 143.444685 145.444685) (end 141.224101 143.224101) (width 0.4) (layer B.Cu) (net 12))
 (segment (start 141.224101 143.224101) (end 141.224101 126.775899) (width 0.4) (layer B.Cu) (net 12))
 (segment (start 141.224101 126.775899) (end 142 126) (width 0.4) (layer B.Cu) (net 12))
 (via (at 142 126) (size 0.6) (drill 0.4) (layers F.Cu B.Cu) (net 12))
 (segment (start 140.2511 126) (end 142 126) (width 0.4) (layer F.Cu) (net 12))
 (segment (start 148.835503 137.92546) (end 148.411239 137.92546) (width 0.4) (layer B.Cu) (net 13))
 (segment (start 154 135.5) (end 151.57454 137.92546) (width 0.4) (layer B.Cu) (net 13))
 (segment (start 151.57454 137.92546) (end 148.835503 137.92546) (width 0.4) (layer B.Cu) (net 13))
 (segment (start 148.11124 138.225459) (end 148.411239 137.92546) (width 0.4) (layer F.Cu) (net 13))
 (segment (start 147.73 138.606699) (end 148.11124 138.225459) (width 0.4) (layer F.Cu) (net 13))
 (segment (start 147.73 140.75) (end 147.73 138.606699) (width 0.4) (layer F.Cu) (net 13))
 (via (at 148.411239 137.92546) (size 0.6) (drill 0.4) (layers F.Cu B.Cu) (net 13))
 (segment (start 153.550001 135.050001) (end 154 135.5) (width 0.4) (layer F.Cu) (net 13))
 (via (at 154 135.5) (size 0.6) (drill 0.4) (layers F.Cu B.Cu) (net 13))
 (segment (start 156.7511 116) (end 155.8511 116) (width 0.4) (layer F.Cu) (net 13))
 (segment (start 155.8511 116) (end 153.550001 118.301099) (width 0.4) (layer F.Cu) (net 13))
 (segment (start 153.550001 118.301099) (end 153.550001 135.050001) (width 0.4) (layer F.Cu) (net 13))
 (segment (start 151 136) (end 149.007759 136) (width 0.4) (layer B.Cu) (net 14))
 (segment (start 149.007759 136) (end 143.982263 141.025496) (width 0.4) (layer B.Cu) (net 14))
 (segment (start 143.982263 141.025496) (end 143.451873 141.025496) (width 0.4) (layer B.Cu) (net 14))
 (segment (start 143.451873 141.025496) (end 143.027609 141.025496) (width 0.4) (layer B.Cu) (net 14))
 (segment (start 143.027609 141.44976) (end 143.027609 141.025496) (width 0.4) (layer F.Cu) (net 14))
 (segment (start 146.46 145.25) (end 145.31 145.25) (width 0.4) (layer F.Cu) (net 14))
 (segment (start 143.027609 142.967609) (end 143.027609 141.44976) (width 0.4) (layer F.Cu) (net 14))
 (segment (start 145.31 145.25) (end 143.027609 142.967609) (width 0.4) (layer F.Cu) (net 14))
 (via (at 143.027609 141.025496) (size 0.6) (drill 0.4) (layers F.Cu B.Cu) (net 14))
 (segment (start 151.449999 135.550001) (end 151 136) (width 0.4) (layer F.Cu) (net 14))
 (via (at 151 136) (size 0.6) (drill 0.4) (layers F.Cu B.Cu) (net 14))
 (segment (start 156.7511 114) (end 155.8511 114) (width 0.4) (layer F.Cu) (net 14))
 (segment (start 155.8511 114) (end 151.449999 118.401101) (width 0.4) (layer F.Cu) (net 14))
 (segment (start 151.449999 118.401101) (end 151.449999 135.550001) (width 0.4) (layer F.Cu) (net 14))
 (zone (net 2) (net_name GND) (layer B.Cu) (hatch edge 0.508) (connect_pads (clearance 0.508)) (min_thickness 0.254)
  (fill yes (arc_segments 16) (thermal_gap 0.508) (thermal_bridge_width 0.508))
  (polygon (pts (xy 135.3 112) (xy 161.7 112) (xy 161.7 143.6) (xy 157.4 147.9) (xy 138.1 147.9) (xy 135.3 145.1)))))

